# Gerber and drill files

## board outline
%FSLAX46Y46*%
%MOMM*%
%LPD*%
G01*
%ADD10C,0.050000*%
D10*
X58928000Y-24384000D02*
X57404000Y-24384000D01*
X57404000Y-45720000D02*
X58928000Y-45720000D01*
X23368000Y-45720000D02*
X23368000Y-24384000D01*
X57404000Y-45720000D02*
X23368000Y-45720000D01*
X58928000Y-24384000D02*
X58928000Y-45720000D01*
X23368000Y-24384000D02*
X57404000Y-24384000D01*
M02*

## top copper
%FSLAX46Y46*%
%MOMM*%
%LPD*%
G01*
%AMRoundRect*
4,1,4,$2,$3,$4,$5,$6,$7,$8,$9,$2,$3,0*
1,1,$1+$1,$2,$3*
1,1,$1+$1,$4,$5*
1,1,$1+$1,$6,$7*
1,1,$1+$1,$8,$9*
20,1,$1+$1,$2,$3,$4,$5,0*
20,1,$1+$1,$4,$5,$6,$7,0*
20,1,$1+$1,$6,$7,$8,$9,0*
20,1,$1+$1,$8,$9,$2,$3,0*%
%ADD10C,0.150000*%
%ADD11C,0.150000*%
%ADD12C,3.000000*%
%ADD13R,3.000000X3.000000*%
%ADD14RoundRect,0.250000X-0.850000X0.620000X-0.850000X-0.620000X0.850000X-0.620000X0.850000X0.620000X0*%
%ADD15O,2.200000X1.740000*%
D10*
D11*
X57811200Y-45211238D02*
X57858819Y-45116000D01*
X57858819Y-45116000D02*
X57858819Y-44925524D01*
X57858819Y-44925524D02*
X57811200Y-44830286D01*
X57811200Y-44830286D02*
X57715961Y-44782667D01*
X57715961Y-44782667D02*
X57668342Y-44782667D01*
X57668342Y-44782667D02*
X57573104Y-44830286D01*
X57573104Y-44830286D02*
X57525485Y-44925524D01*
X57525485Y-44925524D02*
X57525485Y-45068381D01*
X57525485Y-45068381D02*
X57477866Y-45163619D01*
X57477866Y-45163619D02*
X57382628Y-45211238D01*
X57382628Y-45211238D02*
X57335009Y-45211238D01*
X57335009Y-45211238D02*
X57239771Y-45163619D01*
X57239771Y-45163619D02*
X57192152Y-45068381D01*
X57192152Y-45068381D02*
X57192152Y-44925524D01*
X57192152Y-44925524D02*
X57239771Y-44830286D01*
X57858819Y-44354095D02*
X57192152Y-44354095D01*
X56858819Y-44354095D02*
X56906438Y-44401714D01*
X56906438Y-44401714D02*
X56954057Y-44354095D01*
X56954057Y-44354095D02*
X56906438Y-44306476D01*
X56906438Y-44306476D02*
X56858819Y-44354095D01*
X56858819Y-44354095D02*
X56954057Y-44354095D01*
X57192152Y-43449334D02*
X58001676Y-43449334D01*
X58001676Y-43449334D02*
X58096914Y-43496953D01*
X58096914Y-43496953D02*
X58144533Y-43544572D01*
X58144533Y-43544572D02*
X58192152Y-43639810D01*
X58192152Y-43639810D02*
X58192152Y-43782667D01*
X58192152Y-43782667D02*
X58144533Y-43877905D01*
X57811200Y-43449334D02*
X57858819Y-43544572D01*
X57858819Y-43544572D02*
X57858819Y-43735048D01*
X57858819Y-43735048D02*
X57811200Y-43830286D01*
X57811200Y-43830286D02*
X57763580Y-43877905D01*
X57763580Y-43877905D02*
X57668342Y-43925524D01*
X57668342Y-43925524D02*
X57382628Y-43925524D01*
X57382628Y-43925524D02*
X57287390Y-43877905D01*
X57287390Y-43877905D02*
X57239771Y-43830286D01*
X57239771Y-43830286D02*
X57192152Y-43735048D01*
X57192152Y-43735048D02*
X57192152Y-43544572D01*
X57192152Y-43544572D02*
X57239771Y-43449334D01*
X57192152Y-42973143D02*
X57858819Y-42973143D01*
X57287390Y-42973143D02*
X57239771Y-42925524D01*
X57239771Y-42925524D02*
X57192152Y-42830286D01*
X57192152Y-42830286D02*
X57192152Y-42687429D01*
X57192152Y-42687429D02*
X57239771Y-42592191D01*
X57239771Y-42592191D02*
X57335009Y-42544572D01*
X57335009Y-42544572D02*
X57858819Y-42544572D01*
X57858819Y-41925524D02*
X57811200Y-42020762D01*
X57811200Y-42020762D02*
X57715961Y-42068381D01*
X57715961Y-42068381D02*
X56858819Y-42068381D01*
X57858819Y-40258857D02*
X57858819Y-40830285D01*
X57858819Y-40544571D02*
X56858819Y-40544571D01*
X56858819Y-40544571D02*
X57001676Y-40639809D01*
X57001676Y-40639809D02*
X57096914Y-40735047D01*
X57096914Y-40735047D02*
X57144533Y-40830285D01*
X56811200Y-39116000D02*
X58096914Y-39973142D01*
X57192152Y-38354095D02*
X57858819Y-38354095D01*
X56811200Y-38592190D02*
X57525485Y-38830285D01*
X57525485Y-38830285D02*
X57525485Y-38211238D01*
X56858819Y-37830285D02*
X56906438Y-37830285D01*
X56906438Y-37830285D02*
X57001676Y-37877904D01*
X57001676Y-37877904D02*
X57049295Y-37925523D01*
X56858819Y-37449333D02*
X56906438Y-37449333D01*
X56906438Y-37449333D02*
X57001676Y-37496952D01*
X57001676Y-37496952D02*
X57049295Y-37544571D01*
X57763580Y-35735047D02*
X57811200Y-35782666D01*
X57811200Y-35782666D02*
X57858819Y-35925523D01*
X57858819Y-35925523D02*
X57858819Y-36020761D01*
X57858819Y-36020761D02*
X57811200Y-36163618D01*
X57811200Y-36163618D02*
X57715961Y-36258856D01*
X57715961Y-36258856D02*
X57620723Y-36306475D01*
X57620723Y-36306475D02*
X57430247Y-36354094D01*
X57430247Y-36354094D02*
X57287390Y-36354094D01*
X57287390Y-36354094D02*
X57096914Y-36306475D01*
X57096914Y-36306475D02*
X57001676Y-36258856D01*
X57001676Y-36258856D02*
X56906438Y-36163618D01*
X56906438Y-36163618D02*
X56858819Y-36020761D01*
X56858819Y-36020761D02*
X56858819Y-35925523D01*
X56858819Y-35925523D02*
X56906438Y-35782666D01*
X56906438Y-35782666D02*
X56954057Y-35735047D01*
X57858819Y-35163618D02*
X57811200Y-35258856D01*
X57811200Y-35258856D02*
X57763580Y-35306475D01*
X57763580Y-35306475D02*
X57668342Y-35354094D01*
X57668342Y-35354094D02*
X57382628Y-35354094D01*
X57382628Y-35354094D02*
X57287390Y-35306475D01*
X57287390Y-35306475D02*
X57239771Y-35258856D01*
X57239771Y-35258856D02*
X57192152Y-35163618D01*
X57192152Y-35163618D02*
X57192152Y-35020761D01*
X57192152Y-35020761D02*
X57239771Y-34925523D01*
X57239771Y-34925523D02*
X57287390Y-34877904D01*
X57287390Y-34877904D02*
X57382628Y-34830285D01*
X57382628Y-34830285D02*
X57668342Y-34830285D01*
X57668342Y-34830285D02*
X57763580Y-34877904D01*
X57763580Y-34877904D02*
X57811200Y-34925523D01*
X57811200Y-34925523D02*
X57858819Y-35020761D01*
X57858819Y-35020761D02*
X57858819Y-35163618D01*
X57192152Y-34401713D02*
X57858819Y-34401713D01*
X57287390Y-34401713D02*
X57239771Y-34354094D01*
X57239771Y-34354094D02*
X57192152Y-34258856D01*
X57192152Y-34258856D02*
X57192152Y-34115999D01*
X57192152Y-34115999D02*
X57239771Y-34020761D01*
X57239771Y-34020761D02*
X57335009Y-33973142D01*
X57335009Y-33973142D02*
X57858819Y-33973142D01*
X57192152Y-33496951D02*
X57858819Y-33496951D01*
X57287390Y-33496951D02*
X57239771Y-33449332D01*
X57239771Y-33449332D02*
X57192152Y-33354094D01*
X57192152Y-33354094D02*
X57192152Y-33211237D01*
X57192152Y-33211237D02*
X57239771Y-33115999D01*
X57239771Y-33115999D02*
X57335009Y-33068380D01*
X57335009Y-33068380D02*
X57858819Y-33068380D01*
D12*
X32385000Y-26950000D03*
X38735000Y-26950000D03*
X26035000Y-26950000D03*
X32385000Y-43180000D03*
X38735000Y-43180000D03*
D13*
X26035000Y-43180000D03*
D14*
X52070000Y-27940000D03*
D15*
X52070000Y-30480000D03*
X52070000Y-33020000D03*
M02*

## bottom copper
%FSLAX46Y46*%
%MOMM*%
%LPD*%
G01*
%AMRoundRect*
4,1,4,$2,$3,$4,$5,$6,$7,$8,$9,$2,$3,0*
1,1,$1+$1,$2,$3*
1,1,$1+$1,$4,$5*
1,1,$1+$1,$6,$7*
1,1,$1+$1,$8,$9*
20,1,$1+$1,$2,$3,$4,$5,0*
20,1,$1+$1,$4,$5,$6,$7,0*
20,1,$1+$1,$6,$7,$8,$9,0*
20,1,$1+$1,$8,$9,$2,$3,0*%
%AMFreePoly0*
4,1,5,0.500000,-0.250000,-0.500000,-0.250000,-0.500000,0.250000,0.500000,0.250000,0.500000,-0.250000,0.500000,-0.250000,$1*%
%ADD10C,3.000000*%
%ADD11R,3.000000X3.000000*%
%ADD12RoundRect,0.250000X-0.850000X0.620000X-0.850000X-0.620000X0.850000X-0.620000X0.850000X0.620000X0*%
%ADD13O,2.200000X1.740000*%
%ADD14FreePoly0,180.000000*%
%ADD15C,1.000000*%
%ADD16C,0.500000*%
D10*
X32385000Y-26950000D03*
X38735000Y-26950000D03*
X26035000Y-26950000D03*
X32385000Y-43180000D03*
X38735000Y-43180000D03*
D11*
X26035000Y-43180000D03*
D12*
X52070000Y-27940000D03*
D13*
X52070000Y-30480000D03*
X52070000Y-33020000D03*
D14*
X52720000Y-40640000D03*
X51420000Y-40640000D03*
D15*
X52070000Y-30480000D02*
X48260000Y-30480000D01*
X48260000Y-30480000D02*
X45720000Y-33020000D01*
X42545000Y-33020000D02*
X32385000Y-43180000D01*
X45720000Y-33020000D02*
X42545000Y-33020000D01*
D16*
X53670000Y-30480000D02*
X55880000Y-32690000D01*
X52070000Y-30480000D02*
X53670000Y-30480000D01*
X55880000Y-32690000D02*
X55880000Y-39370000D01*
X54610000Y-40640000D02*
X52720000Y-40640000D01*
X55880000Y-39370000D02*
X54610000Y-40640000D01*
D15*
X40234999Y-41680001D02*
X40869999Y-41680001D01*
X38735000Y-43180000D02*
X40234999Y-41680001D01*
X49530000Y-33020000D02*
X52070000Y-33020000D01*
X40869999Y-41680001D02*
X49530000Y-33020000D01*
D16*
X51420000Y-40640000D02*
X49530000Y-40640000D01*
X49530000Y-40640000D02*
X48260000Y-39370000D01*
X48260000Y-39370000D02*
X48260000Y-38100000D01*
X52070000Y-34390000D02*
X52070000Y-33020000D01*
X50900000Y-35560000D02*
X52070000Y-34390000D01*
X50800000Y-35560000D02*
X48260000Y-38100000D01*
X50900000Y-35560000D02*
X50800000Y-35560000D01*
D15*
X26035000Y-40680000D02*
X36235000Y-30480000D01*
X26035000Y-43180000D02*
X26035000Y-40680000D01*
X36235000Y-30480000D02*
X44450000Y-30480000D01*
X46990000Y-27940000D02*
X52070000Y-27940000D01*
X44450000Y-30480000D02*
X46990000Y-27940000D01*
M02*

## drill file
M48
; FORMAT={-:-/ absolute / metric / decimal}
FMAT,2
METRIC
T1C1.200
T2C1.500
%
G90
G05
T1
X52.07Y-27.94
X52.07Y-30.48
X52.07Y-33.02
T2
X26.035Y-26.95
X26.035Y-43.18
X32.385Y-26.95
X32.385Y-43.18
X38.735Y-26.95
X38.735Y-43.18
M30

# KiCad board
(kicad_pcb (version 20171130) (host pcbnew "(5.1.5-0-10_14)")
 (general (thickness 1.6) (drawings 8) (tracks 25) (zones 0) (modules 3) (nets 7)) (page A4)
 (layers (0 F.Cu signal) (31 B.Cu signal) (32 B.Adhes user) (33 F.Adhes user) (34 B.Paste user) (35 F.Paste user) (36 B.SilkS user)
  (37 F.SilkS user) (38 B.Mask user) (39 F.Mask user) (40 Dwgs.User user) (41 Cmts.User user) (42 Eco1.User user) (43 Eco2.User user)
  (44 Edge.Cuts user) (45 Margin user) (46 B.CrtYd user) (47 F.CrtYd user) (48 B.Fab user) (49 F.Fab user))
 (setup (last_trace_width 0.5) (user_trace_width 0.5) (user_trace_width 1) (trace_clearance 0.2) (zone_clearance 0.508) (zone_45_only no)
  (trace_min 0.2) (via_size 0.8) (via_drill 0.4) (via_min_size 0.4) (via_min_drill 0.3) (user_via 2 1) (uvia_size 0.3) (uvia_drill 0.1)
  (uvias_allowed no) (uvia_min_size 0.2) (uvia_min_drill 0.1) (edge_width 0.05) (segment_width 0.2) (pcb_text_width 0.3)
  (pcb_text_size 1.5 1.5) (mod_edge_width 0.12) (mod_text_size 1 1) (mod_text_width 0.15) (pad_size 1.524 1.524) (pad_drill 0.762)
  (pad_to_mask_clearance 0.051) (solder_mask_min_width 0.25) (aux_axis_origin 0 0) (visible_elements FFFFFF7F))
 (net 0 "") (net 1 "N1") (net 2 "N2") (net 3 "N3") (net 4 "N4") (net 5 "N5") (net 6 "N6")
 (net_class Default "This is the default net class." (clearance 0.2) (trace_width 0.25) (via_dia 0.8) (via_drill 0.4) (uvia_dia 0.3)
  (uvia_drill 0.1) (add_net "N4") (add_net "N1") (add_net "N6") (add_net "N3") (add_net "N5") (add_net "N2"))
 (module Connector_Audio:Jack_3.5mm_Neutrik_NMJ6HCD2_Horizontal (layer F.Cu) (at 38.735 43.18 180)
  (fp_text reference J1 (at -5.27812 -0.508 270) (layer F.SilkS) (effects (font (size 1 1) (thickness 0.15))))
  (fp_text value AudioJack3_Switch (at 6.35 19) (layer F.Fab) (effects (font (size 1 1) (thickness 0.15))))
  (pad RN thru_hole circle (at 6.35 16.23 180) (size 3 3) (drill 1.5) (layers *.Cu *.Mask) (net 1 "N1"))
  (pad TN thru_hole circle (at 0 16.23 180) (size 3 3) (drill 1.5) (layers *.Cu *.Mask) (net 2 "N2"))
  (pad SN thru_hole circle (at 12.7 16.23 180) (size 3 3) (drill 1.5) (layers *.Cu *.Mask) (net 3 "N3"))
  (pad R thru_hole circle (at 6.35 0 180) (size 3 3) (drill 1.5) (layers *.Cu *.Mask) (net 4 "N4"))
  (pad T thru_hole circle (at 0 0 180) (size 3 3) (drill 1.5) (layers *.Cu *.Mask) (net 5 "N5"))
  (pad S thru_hole rect (at 12.7 0 180) (size 3 3) (drill 1.5) (layers *.Cu *.Mask) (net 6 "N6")))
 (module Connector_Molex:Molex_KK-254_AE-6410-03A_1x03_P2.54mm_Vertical (layer F.Cu) (at 52.07 27.94 270)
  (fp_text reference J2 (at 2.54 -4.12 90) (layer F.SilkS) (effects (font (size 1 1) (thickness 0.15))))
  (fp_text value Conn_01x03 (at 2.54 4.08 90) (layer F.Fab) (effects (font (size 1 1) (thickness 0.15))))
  (pad 1 thru_hole roundrect (at 0 0 270) (size 1.74 2.2) (drill 1.2) (layers *.Cu *.Mask) (roundrect_rratio 0.143678) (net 6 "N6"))
  (pad 2 thru_hole oval (at 2.54 0 270) (size 1.74 2.2) (drill 1.2) (layers *.Cu *.Mask) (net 4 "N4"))
  (pad 3 thru_hole oval (at 5.08 0 270) (size 1.74 2.2) (drill 1.2) (layers *.Cu *.Mask) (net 5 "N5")))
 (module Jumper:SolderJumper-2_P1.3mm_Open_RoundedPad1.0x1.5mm (layer B.Cu) (at 52.07 40.64 180)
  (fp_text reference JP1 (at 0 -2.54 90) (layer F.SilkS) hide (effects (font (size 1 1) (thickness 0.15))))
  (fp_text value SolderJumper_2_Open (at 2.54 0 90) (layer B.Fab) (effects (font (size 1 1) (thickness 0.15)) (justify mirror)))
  (pad 1 smd custom (at -0.65 0 180) (size 1 0.5) (layers B.Cu B.Mask) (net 4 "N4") (zone_connect 2)
   (options (clearance outline) (anchor rect)) (primitives))
  (pad 2 smd custom (at 0.65 0 180) (size 1 0.5) (layers B.Cu B.Mask) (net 5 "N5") (zone_connect 2)
   (options (clearance outline) (anchor rect)) (primitives)))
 (gr_line (start 58.928 24.384) (end 57.404 24.384) (layer Edge.Cuts) (width 0.05))
 (gr_line (start 57.404 45.72) (end 58.928 45.72) (layer Edge.Cuts) (width 0.05))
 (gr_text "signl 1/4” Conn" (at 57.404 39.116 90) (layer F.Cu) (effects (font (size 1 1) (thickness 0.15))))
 (gr_line (start 23.368 45.72) (end 23.368 24.384) (layer Edge.Cuts) (width 0.05))
 (gr_line (start 57.404 45.72) (end 23.368 45.72) (layer Edge.Cuts) (width 0.05))
 (gr_line (start 58.928 24.384) (end 58.928 45.72) (layer Edge.Cuts) (width 0.05))
 (gr_line (start 23.368 24.384) (end 57.404 24.384) (layer Edge.Cuts) (width 0.05))
 (segment (start 52.07 30.48) (end 48.26 30.48) (width 1) (layer B.Cu) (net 4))
 (segment (start 48.26 30.48) (end 45.72 33.02) (width 1) (layer B.Cu) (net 4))
 (segment (start 42.545 33.02) (end 32.385 43.18) (width 1) (layer B.Cu) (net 4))
 (segment (start 45.72 33.02) (end 42.545 33.02) (width 1) (layer B.Cu) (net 4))
 (segment (start 53.67 30.48) (end 55.88 32.69) (width 0.5) (layer B.Cu) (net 4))
 (segment (start 52.07 30.48) (end 53.67 30.48) (width 0.5) (layer B.Cu) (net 4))
 (segment (start 55.88 32.69) (end 55.88 39.37) (width 0.5) (layer B.Cu) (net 4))
 (segment (start 54.61 40.64) (end 52.72 40.64) (width 0.5) (layer B.Cu) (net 4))
 (segment (start 55.88 39.37) (end 54.61 40.64) (width 0.5) (layer B.Cu) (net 4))
 (segment (start 40.234999 41.680001) (end 40.869999 41.680001) (width 1) (layer B.Cu) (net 5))
 (segment (start 38.735 43.18) (end 40.234999 41.680001) (width 1) (layer B.Cu) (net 5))
 (segment (start 49.53 33.02) (end 52.07 33.02) (width 1) (layer B.Cu) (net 5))
 (segment (start 40.869999 41.680001) (end 49.53 33.02) (width 1) (layer B.Cu) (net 5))
 (segment (start 51.42 40.64) (end 49.53 40.64) (width 0.5) (layer B.Cu) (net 5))
 (segment (start 49.53 40.64) (end 48.26 39.37) (width 0.5) (layer B.Cu) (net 5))
 (segment (start 48.26 39.37) (end 48.26 38.1) (width 0.5) (layer B.Cu) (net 5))
 (segment (start 52.07 34.39) (end 52.07 33.02) (width 0.5) (layer B.Cu) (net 5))
 (segment (start 50.9 35.56) (end 52.07 34.39) (width 0.5) (layer B.Cu) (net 5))
 (segment (start 50.8 35.56) (end 48.26 38.1) (width 0.5) (layer B.Cu) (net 5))
 (segment (start 50.9 35.56) (end 50.8 35.56) (width 0.5) (layer B.Cu) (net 5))
 (segment (start 26.035 40.68) (end 36.235 30.48) (width 1) (layer B.Cu) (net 6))
 (segment (start 26.035 43.18) (end 26.035 40.68) (width 1) (layer B.Cu) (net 6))
 (segment (start 36.235 30.48) (end 44.45 30.48) (width 1) (layer B.Cu) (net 6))
 (segment (start 46.99 27.94) (end 52.07 27.94) (width 1) (layer B.Cu) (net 6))
 (segment (start 44.45 30.48) (end 46.99 27.94) (width 1) (layer B.Cu) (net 6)))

